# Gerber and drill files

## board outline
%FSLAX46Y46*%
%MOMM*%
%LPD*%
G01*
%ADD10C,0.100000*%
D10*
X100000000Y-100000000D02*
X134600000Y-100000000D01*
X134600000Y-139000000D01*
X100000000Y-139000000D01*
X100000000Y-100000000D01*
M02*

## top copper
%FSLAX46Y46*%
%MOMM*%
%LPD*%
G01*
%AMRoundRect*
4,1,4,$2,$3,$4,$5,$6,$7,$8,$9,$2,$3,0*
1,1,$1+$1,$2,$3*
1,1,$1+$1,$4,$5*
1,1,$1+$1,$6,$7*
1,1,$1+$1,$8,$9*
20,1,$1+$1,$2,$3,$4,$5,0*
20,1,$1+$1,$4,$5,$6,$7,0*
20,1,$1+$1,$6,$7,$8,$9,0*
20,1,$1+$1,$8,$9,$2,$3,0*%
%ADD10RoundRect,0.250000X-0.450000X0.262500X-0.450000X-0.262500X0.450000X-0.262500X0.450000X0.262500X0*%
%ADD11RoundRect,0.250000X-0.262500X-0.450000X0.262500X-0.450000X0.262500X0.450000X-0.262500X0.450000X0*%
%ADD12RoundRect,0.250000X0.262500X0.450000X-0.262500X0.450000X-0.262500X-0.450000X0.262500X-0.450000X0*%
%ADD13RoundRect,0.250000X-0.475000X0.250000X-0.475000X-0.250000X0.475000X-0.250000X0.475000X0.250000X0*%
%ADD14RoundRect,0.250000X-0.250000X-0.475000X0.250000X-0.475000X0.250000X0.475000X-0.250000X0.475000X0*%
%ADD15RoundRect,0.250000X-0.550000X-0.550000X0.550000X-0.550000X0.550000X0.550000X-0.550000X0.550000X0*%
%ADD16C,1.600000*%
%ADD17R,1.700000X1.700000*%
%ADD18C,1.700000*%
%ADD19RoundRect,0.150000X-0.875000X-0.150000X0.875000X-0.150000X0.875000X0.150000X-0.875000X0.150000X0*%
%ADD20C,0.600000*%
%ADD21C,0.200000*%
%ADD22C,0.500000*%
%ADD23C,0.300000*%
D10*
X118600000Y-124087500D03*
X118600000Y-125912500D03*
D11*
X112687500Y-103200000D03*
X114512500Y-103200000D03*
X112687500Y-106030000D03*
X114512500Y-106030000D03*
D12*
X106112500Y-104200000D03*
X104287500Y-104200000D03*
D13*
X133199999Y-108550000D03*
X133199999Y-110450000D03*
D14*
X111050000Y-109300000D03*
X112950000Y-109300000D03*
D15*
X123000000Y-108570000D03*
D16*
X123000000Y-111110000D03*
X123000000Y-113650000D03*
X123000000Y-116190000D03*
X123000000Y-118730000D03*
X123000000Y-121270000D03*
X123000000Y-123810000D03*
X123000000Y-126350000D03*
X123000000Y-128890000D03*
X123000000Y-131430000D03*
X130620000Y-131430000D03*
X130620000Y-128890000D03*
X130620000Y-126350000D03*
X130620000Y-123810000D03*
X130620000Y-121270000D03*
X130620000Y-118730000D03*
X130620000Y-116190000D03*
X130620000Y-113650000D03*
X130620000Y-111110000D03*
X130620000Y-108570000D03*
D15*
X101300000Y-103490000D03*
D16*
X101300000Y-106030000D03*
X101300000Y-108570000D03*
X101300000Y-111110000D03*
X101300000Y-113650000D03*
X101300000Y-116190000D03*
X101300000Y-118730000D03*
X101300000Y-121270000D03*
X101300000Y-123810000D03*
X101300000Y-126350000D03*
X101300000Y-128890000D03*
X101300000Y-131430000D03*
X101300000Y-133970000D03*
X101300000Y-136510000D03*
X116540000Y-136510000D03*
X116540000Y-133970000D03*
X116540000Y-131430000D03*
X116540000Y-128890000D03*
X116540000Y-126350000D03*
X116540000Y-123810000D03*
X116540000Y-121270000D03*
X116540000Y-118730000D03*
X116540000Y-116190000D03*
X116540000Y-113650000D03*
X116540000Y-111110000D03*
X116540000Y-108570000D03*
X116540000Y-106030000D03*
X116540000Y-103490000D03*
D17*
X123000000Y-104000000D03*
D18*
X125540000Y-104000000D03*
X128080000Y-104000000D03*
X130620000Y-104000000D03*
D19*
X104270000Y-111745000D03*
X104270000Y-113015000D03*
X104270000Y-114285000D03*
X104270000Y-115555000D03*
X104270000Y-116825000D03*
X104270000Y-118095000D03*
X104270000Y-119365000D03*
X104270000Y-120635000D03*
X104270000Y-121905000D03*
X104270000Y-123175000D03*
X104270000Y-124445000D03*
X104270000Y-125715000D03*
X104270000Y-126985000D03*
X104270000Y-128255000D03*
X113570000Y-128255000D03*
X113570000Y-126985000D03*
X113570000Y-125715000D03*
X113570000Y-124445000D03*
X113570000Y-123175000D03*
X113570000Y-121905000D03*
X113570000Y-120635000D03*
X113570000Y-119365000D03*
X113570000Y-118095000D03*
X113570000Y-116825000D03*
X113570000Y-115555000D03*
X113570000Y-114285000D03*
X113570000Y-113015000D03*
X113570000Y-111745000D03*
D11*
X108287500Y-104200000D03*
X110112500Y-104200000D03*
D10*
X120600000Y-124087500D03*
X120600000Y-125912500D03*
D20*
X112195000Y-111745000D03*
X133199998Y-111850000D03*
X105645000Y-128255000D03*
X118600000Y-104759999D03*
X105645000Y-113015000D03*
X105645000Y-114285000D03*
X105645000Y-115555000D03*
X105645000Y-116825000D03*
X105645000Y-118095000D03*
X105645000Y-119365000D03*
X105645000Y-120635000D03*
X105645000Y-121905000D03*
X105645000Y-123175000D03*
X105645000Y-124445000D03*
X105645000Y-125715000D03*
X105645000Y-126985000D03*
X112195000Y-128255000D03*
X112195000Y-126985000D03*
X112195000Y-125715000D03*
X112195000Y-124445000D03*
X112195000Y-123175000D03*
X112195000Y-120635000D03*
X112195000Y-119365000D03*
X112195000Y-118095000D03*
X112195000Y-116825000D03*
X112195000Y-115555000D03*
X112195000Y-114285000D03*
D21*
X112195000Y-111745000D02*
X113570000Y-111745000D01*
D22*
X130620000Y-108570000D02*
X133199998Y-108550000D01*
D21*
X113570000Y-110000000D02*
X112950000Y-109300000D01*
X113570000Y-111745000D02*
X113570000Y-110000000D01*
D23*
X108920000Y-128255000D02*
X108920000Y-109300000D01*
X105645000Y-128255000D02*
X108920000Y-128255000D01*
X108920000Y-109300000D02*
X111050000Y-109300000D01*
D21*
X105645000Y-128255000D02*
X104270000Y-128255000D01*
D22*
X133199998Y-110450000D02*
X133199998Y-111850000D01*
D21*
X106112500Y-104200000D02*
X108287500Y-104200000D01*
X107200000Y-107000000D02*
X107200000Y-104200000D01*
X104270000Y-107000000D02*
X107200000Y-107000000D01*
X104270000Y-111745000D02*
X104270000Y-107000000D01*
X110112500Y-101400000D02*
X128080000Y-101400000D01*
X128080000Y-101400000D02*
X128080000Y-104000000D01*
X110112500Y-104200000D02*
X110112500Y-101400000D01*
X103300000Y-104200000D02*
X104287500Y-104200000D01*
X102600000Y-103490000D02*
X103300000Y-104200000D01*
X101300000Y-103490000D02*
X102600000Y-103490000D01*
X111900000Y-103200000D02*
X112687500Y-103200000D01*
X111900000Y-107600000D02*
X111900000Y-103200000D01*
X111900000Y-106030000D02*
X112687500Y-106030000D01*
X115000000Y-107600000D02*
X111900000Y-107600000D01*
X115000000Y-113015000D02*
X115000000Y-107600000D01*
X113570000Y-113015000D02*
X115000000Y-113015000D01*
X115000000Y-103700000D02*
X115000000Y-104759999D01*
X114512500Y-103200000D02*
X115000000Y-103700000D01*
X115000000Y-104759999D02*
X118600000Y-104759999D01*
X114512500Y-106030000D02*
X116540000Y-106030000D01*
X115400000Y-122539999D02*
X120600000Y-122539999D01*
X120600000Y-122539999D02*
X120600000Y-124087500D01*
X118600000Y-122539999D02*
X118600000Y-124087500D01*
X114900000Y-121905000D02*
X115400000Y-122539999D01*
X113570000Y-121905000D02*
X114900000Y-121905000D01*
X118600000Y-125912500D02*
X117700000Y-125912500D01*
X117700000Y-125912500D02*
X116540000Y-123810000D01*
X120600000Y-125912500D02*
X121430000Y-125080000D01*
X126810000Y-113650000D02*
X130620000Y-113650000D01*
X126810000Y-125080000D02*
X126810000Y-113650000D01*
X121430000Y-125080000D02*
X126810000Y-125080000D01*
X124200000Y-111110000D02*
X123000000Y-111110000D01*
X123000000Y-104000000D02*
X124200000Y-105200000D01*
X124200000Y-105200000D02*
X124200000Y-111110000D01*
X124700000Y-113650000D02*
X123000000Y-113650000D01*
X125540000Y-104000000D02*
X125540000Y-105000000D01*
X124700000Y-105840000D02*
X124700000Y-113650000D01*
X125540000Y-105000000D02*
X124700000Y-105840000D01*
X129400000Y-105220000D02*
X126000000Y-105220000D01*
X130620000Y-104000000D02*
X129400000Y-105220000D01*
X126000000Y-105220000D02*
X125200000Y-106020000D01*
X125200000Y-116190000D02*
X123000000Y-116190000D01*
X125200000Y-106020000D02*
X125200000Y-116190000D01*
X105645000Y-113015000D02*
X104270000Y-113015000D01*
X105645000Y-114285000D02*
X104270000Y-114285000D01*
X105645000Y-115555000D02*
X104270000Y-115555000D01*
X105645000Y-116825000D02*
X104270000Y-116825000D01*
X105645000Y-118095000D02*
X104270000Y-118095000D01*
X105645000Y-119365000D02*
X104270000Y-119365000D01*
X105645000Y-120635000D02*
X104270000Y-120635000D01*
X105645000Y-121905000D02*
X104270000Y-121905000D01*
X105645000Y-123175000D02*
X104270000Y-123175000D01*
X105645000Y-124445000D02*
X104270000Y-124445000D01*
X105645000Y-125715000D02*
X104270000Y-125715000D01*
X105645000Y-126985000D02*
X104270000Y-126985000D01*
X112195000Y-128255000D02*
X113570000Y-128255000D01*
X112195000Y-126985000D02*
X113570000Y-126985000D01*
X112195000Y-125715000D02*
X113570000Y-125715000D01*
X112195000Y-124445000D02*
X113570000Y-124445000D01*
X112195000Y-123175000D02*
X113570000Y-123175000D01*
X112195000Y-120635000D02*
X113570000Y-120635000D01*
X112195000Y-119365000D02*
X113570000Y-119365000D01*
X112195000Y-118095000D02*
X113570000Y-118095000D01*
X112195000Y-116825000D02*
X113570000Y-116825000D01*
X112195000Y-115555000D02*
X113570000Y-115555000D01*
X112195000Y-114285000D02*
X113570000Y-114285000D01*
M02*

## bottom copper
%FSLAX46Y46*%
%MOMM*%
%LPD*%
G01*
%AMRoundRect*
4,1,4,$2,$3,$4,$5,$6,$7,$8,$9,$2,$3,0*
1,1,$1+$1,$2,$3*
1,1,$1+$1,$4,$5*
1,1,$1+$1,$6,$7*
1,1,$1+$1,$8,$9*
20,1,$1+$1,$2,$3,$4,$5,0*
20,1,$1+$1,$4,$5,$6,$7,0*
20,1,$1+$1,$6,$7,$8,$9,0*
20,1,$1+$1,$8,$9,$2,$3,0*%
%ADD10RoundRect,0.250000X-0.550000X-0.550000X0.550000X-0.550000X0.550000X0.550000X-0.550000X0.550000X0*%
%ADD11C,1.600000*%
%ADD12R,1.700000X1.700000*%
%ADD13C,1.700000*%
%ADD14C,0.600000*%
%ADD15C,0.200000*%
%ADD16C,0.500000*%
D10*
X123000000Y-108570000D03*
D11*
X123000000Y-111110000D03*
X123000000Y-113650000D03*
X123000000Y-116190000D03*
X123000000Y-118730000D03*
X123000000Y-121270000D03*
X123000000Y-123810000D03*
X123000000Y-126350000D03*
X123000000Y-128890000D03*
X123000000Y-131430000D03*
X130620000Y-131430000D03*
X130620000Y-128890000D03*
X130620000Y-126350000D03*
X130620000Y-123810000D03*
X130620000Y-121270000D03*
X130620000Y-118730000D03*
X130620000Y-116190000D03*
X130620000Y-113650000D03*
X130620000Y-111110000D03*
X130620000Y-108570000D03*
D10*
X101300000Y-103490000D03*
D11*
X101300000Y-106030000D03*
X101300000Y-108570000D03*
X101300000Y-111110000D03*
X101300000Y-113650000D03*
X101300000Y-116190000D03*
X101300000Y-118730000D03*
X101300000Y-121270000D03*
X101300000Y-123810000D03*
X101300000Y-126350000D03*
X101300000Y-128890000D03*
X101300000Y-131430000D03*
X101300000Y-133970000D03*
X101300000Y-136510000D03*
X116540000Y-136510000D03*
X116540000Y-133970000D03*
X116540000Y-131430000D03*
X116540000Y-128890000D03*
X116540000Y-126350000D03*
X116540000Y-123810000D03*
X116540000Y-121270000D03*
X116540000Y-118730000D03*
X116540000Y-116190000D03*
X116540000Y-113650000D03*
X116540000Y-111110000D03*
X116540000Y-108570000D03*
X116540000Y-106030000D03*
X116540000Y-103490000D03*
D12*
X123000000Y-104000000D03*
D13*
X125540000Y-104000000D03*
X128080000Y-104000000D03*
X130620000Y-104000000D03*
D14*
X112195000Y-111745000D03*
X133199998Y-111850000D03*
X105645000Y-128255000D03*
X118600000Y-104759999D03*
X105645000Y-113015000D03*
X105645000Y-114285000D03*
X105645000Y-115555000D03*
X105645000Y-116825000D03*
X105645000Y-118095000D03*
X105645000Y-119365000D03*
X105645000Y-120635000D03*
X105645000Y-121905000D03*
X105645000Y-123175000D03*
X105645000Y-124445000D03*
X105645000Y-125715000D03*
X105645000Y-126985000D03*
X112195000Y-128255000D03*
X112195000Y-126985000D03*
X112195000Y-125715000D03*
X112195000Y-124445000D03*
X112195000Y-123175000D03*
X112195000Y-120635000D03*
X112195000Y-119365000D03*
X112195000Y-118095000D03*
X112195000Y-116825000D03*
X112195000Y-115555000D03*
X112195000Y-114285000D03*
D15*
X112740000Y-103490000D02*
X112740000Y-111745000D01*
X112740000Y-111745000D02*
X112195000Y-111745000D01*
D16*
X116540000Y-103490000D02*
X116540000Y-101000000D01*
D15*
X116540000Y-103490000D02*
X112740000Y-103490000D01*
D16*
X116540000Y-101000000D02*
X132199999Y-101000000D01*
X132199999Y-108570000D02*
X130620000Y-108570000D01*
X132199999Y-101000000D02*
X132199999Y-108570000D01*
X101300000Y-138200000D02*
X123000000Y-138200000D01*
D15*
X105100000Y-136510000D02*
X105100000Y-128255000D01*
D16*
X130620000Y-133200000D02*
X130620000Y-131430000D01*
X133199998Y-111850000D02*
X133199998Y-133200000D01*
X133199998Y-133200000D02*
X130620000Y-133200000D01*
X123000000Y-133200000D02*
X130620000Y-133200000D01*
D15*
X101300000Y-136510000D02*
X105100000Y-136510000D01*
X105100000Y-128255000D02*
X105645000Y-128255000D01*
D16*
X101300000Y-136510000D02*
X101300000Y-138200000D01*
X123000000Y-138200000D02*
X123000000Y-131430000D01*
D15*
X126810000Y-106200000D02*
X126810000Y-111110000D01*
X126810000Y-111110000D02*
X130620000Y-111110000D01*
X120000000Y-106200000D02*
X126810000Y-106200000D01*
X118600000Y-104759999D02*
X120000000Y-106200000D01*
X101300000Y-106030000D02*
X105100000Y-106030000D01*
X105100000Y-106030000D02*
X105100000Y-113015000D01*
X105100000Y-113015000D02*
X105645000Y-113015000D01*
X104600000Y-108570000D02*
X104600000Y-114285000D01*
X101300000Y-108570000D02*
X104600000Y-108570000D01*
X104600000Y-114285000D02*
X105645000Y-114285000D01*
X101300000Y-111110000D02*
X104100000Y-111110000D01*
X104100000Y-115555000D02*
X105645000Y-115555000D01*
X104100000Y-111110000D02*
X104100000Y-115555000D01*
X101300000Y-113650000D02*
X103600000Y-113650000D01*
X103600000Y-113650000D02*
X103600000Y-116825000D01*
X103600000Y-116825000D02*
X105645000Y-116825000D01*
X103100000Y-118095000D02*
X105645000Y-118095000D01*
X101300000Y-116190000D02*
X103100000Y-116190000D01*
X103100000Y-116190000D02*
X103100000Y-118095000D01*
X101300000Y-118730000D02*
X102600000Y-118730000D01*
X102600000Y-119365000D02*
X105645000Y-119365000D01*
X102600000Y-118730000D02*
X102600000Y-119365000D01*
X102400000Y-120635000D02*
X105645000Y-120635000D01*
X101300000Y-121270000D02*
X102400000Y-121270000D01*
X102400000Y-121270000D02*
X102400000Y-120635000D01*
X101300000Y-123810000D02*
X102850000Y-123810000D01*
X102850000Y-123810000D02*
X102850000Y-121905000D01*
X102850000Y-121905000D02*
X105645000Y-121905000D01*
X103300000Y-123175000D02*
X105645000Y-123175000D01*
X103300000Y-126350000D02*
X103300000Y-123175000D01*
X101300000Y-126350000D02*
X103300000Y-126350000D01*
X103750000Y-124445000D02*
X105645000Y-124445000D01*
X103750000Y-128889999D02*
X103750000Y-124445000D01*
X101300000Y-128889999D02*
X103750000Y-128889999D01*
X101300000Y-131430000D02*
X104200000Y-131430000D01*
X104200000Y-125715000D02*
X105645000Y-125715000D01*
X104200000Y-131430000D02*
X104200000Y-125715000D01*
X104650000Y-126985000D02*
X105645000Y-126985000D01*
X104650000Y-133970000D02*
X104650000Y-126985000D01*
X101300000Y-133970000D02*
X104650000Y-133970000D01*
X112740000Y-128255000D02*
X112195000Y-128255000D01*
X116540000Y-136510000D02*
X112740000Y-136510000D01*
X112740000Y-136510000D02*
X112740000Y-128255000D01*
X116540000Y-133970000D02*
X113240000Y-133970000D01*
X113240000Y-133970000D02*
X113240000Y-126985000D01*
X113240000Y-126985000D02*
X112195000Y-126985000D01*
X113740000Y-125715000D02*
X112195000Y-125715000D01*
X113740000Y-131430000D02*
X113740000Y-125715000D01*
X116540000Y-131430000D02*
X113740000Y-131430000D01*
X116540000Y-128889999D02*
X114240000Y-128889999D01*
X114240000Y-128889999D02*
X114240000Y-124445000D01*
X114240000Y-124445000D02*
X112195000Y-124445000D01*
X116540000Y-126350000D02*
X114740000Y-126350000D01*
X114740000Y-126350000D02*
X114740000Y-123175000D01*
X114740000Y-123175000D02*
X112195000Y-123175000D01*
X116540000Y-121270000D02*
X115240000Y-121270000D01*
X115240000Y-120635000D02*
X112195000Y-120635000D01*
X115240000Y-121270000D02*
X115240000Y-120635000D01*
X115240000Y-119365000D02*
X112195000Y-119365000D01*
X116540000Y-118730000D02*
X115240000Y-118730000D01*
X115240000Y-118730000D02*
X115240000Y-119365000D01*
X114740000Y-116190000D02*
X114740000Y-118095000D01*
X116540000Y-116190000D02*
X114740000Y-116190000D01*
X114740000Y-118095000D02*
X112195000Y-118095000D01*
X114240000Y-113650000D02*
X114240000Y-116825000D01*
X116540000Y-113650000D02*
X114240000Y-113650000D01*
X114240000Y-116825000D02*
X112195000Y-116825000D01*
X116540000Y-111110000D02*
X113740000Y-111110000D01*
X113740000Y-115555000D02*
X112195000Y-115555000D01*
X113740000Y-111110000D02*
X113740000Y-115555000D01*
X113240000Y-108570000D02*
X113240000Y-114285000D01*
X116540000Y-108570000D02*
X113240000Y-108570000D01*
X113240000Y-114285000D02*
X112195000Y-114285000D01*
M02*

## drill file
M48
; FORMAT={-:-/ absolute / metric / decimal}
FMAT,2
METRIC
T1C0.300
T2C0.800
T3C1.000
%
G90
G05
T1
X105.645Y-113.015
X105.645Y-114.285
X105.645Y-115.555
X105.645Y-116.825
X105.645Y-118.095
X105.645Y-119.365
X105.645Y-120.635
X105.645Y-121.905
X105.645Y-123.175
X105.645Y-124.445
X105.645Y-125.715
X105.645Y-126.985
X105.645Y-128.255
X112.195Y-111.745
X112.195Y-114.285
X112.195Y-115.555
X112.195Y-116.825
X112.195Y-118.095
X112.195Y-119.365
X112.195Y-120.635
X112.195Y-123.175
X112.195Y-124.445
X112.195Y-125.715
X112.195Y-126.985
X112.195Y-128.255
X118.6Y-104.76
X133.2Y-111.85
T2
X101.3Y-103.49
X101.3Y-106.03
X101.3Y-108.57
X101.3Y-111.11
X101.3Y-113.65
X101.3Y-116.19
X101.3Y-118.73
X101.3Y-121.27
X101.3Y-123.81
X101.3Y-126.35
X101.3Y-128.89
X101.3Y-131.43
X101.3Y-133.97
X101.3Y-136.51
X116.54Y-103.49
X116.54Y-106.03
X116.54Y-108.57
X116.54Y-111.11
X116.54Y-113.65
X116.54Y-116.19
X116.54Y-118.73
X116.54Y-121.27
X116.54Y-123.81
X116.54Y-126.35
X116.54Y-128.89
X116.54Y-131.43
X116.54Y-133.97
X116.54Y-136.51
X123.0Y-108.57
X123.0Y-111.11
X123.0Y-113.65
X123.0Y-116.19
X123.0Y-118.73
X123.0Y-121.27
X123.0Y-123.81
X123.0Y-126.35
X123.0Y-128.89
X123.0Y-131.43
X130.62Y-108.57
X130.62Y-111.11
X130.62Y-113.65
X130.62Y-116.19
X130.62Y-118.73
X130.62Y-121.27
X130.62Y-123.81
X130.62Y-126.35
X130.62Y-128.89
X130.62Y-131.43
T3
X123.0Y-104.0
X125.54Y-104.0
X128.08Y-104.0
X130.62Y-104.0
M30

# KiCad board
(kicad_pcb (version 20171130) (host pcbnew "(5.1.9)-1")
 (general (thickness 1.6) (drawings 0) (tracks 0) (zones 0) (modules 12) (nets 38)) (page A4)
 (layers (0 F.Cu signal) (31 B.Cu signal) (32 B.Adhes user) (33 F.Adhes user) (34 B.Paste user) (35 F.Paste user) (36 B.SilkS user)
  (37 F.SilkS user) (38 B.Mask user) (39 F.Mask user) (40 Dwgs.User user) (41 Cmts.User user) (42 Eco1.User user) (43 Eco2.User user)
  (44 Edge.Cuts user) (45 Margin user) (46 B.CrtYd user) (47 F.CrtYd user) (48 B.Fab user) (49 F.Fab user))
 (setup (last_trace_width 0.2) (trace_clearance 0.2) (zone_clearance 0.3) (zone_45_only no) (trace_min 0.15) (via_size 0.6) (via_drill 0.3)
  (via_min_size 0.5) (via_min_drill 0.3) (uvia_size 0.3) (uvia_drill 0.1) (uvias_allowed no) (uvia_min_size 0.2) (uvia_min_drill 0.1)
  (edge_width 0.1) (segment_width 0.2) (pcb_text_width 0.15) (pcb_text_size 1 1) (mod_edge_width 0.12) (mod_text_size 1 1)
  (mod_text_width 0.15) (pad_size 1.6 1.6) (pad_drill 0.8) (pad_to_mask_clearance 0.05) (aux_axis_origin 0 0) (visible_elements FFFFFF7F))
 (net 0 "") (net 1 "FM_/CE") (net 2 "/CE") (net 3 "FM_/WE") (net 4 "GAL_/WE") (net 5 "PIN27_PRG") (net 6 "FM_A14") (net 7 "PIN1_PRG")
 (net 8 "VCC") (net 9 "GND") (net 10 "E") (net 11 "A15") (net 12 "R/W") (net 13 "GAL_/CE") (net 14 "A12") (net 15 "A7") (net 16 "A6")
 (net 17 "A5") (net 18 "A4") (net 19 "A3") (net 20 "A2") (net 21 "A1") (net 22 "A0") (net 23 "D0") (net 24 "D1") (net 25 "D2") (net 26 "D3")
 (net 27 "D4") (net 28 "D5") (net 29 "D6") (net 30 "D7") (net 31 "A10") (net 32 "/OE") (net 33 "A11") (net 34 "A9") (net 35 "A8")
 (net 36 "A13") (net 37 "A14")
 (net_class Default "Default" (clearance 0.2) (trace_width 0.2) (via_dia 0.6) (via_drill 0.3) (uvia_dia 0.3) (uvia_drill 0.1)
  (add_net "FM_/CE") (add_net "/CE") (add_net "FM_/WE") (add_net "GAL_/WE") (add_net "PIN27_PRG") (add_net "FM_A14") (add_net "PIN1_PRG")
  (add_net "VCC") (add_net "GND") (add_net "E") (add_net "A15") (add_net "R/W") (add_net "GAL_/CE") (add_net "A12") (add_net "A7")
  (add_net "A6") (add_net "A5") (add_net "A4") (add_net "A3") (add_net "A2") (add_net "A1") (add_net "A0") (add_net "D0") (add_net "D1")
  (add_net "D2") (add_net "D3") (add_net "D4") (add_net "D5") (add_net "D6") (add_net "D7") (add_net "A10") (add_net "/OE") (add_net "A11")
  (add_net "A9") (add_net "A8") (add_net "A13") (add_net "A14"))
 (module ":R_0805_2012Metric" (layer F.Cu) (at 118.6 125 -90)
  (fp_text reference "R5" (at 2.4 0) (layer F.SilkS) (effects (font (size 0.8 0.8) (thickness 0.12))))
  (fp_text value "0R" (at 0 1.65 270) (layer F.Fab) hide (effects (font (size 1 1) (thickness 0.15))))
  (pad "1" smd roundrect (at -0.9125 0 270) (size 1.025 1.4) (layers F.Cu F.Paste F.Mask) (roundrect_rratio 0.2439) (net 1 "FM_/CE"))
  (pad "2" smd roundrect (at 0.9125 0 270) (size 1.025 1.4) (layers F.Cu F.Paste F.Mask) (roundrect_rratio 0.2439) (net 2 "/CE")))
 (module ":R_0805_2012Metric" (layer F.Cu) (at 113.6 103.2)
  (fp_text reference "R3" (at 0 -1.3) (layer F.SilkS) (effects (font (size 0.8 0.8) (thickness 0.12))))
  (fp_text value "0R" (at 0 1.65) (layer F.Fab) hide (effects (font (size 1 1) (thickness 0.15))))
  (pad "1" smd roundrect (at -0.9125 0) (size 1.025 1.4) (layers F.Cu F.Paste F.Mask) (roundrect_rratio 0.2439) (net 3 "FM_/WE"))
  (pad "2" smd roundrect (at 0.9125 0) (size 1.025 1.4) (layers F.Cu F.Paste F.Mask) (roundrect_rratio 0.2439) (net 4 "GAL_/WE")))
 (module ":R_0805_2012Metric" (layer F.Cu) (at 113.6 106.03)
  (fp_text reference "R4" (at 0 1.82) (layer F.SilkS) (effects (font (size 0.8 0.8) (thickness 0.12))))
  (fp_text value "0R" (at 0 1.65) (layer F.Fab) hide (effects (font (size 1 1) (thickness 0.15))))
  (pad "1" smd roundrect (at -0.9125 0) (size 1.025 1.4) (layers F.Cu F.Paste F.Mask) (roundrect_rratio 0.2439) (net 3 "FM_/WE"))
  (pad "2" smd roundrect (at 0.9125 0) (size 1.025 1.4) (layers F.Cu F.Paste F.Mask) (roundrect_rratio 0.2439) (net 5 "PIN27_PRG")))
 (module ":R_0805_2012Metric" (layer F.Cu) (at 105.2 104.2 180)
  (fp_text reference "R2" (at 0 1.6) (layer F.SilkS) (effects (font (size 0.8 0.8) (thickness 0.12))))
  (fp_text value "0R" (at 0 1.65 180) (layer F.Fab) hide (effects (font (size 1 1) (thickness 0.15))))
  (pad "1" smd roundrect (at -0.9125 0 180) (size 1.025 1.4) (layers F.Cu F.Paste F.Mask) (roundrect_rratio 0.2439) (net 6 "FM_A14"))
  (pad "2" smd roundrect (at 0.9125 0 180) (size 1.025 1.4) (layers F.Cu F.Paste F.Mask) (roundrect_rratio 0.2439) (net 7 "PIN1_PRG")))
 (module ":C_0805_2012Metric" (layer F.Cu) (at 133.2 109.5 -90)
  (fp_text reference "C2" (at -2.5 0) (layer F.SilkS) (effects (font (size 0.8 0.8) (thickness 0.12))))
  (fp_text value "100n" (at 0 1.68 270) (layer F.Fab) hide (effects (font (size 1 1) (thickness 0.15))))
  (pad "1" smd roundrect (at -0.95 0 270) (size 1 1.45) (layers F.Cu F.Paste F.Mask) (roundrect_rratio 0.25) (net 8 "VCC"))
  (pad "2" smd roundrect (at 0.95 0 270) (size 1 1.45) (layers F.Cu F.Paste F.Mask) (roundrect_rratio 0.25) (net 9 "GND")))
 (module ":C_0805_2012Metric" (layer F.Cu) (at 112 109.3)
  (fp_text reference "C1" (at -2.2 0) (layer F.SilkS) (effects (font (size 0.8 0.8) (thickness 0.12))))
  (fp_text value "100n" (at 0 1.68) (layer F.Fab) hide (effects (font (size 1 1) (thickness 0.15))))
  (pad "1" smd roundrect (at -0.95 0) (size 1 1.45) (layers F.Cu F.Paste F.Mask) (roundrect_rratio 0.25) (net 9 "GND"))
  (pad "2" smd roundrect (at 0.95 0) (size 1 1.45) (layers F.Cu F.Paste F.Mask) (roundrect_rratio 0.25) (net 8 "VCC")))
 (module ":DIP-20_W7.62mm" (layer F.Cu) (at 123 108.57)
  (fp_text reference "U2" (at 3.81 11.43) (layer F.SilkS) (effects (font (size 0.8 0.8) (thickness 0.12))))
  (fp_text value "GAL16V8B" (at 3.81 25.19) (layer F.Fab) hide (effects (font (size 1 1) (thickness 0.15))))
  (pad "1" thru_hole roundrect (at 0 0) (size 1.6 1.6) (drill 0.8) (layers *.Cu *.Mask) (roundrect_rratio 0.1562))
  (pad "2" thru_hole circle (at 0 2.54) (size 1.6 1.6) (drill 0.8) (layers *.Cu *.Mask) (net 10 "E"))
  (pad "3" thru_hole circle (at 0 5.08) (size 1.6 1.6) (drill 0.8) (layers *.Cu *.Mask) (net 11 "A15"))
  (pad "4" thru_hole circle (at 0 7.62) (size 1.6 1.6) (drill 0.8) (layers *.Cu *.Mask) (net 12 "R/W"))
  (pad "5" thru_hole circle (at 0 10.16) (size 1.6 1.6) (drill 0.8) (layers *.Cu *.Mask))
  (pad "6" thru_hole circle (at 0 12.7) (size 1.6 1.6) (drill 0.8) (layers *.Cu *.Mask))
  (pad "7" thru_hole circle (at 0 15.24) (size 1.6 1.6) (drill 0.8) (layers *.Cu *.Mask))
  (pad "8" thru_hole circle (at 0 17.78) (size 1.6 1.6) (drill 0.8) (layers *.Cu *.Mask))
  (pad "9" thru_hole circle (at 0 20.32) (size 1.6 1.6) (drill 0.8) (layers *.Cu *.Mask))
  (pad "10" thru_hole circle (at 0 22.86) (size 1.6 1.6) (drill 0.8) (layers *.Cu *.Mask) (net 9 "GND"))
  (pad "11" thru_hole circle (at 7.62 22.86) (size 1.6 1.6) (drill 0.8) (layers *.Cu *.Mask) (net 9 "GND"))
  (pad "12" thru_hole circle (at 7.62 20.32) (size 1.6 1.6) (drill 0.8) (layers *.Cu *.Mask))
  (pad "13" thru_hole circle (at 7.62 17.78) (size 1.6 1.6) (drill 0.8) (layers *.Cu *.Mask))
  (pad "14" thru_hole circle (at 7.62 15.24) (size 1.6 1.6) (drill 0.8) (layers *.Cu *.Mask))
  (pad "15" thru_hole circle (at 7.62 12.7) (size 1.6 1.6) (drill 0.8) (layers *.Cu *.Mask))
  (pad "16" thru_hole circle (at 7.62 10.16) (size 1.6 1.6) (drill 0.8) (layers *.Cu *.Mask))
  (pad "17" thru_hole circle (at 7.62 7.62) (size 1.6 1.6) (drill 0.8) (layers *.Cu *.Mask))
  (pad "18" thru_hole circle (at 7.62 5.08) (size 1.6 1.6) (drill 0.8) (layers *.Cu *.Mask) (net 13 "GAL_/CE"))
  (pad "19" thru_hole circle (at 7.62 2.54) (size 1.6 1.6) (drill 0.8) (layers *.Cu *.Mask) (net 4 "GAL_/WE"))
  (pad "20" thru_hole circle (at 7.62 0) (size 1.6 1.6) (drill 0.8) (layers *.Cu *.Mask) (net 8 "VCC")))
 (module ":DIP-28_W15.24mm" (layer F.Cu) (at 101.3 103.49)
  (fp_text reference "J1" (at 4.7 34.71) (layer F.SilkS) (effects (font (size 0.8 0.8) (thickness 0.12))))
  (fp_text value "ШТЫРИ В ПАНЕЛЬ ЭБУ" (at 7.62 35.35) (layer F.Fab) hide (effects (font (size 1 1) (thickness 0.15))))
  (pad "1" thru_hole roundrect (at 0 0) (size 1.6 1.6) (drill 0.8) (layers *.Cu *.Mask) (roundrect_rratio 0.1562) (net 7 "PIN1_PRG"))
  (pad "2" thru_hole circle (at 0 2.54) (size 1.6 1.6) (drill 0.8) (layers *.Cu *.Mask) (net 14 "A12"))
  (pad "3" thru_hole circle (at 0 5.08) (size 1.6 1.6) (drill 0.8) (layers *.Cu *.Mask) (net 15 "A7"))
  (pad "4" thru_hole circle (at 0 7.62) (size 1.6 1.6) (drill 0.8) (layers *.Cu *.Mask) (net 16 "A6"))
  (pad "5" thru_hole circle (at 0 10.16) (size 1.6 1.6) (drill 0.8) (layers *.Cu *.Mask) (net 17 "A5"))
  (pad "6" thru_hole circle (at 0 12.7) (size 1.6 1.6) (drill 0.8) (layers *.Cu *.Mask) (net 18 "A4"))
  (pad "7" thru_hole circle (at 0 15.24) (size 1.6 1.6) (drill 0.8) (layers *.Cu *.Mask) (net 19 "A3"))
  (pad "8" thru_hole circle (at 0 17.78) (size 1.6 1.6) (drill 0.8) (layers *.Cu *.Mask) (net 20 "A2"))
  (pad "9" thru_hole circle (at 0 20.32) (size 1.6 1.6) (drill 0.8) (layers *.Cu *.Mask) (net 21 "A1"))
  (pad "10" thru_hole circle (at 0 22.86) (size 1.6 1.6) (drill 0.8) (layers *.Cu *.Mask) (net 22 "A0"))
  (pad "11" thru_hole circle (at 0 25.4) (size 1.6 1.6) (drill 0.8) (layers *.Cu *.Mask) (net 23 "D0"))
  (pad "12" thru_hole circle (at 0 27.94) (size 1.6 1.6) (drill 0.8) (layers *.Cu *.Mask) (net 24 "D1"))
  (pad "13" thru_hole circle (at 0 30.48) (size 1.6 1.6) (drill 0.8) (layers *.Cu *.Mask) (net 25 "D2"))
  (pad "14" thru_hole circle (at 0 33.02) (size 1.6 1.6) (drill 0.8) (layers *.Cu *.Mask) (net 9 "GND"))
  (pad "15" thru_hole circle (at 15.24 33.02) (size 1.6 1.6) (drill 0.8) (layers *.Cu *.Mask) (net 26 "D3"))
  (pad "16" thru_hole circle (at 15.24 30.48) (size 1.6 1.6) (drill 0.8) (layers *.Cu *.Mask) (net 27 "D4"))
  (pad "17" thru_hole circle (at 15.24 27.94) (size 1.6 1.6) (drill 0.8) (layers *.Cu *.Mask) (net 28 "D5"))
  (pad "18" thru_hole circle (at 15.24 25.4) (size 1.6 1.6) (drill 0.8) (layers *.Cu *.Mask) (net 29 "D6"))
  (pad "19" thru_hole circle (at 15.24 22.86) (size 1.6 1.6) (drill 0.8) (layers *.Cu *.Mask) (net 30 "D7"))
  (pad "20" thru_hole circle (at 15.24 20.32) (size 1.6 1.6) (drill 0.8) (layers *.Cu *.Mask) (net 2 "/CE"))
  (pad "21" thru_hole circle (at 15.24 17.78) (size 1.6 1.6) (drill 0.8) (layers *.Cu *.Mask) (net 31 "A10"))
  (pad "22" thru_hole circle (at 15.24 15.24) (size 1.6 1.6) (drill 0.8) (layers *.Cu *.Mask) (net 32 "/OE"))
  (pad "23" thru_hole circle (at 15.24 12.7) (size 1.6 1.6) (drill 0.8) (layers *.Cu *.Mask) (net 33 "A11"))
  (pad "24" thru_hole circle (at 15.24 10.16) (size 1.6 1.6) (drill 0.8) (layers *.Cu *.Mask) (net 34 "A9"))
  (pad "25" thru_hole circle (at 15.24 7.62) (size 1.6 1.6) (drill 0.8) (layers *.Cu *.Mask) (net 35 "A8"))
  (pad "26" thru_hole circle (at 15.24 5.08) (size 1.6 1.6) (drill 0.8) (layers *.Cu *.Mask) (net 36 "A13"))
  (pad "27" thru_hole circle (at 15.24 2.54) (size 1.6 1.6) (drill 0.8) (layers *.Cu *.Mask) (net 5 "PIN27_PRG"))
  (pad "28" thru_hole circle (at 15.24 0) (size 1.6 1.6) (drill 0.8) (layers *.Cu *.Mask) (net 8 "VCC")))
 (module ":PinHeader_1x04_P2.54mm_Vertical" (layer F.Cu) (at 123 104 90)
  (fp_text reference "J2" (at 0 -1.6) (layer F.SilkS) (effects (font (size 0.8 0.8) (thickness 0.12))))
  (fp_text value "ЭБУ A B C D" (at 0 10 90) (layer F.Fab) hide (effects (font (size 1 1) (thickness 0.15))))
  (pad "1" thru_hole rect (at 0 0 90) (size 1.7 1.7) (drill 1) (layers *.Cu *.Mask) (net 10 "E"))
  (pad "2" thru_hole circle (at 0 2.54 90) (size 1.7 1.7) (drill 1) (layers *.Cu *.Mask) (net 11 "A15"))
  (pad "3" thru_hole circle (at 0 5.08 90) (size 1.7 1.7) (drill 1) (layers *.Cu *.Mask) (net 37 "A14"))
  (pad "4" thru_hole circle (at 0 7.62 90) (size 1.7 1.7) (drill 1) (layers *.Cu *.Mask) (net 12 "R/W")))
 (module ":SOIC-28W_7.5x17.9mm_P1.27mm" (layer F.Cu) (at 108.92 120)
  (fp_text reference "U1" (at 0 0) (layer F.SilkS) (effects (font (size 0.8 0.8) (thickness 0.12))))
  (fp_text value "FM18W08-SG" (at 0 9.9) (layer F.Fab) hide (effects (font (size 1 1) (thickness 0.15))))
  (pad "1" smd roundrect (at -4.65 -8.255) (size 2.05 0.6) (layers F.Cu F.Paste F.Mask) (roundrect_rratio 0.25) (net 6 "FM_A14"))
  (pad "2" smd roundrect (at -4.65 -6.985) (size 2.05 0.6) (layers F.Cu F.Paste F.Mask) (roundrect_rratio 0.25) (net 14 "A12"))
  (pad "3" smd roundrect (at -4.65 -5.715) (size 2.05 0.6) (layers F.Cu F.Paste F.Mask) (roundrect_rratio 0.25) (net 15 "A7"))
  (pad "4" smd roundrect (at -4.65 -4.445) (size 2.05 0.6) (layers F.Cu F.Paste F.Mask) (roundrect_rratio 0.25) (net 16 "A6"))
  (pad "5" smd roundrect (at -4.65 -3.175) (size 2.05 0.6) (layers F.Cu F.Paste F.Mask) (roundrect_rratio 0.25) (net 17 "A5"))
  (pad "6" smd roundrect (at -4.65 -1.905) (size 2.05 0.6) (layers F.Cu F.Paste F.Mask) (roundrect_rratio 0.25) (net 18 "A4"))
  (pad "7" smd roundrect (at -4.65 -0.635) (size 2.05 0.6) (layers F.Cu F.Paste F.Mask) (roundrect_rratio 0.25) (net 19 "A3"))
  (pad "8" smd roundrect (at -4.65 0.635) (size 2.05 0.6) (layers F.Cu F.Paste F.Mask) (roundrect_rratio 0.25) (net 20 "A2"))
  (pad "9" smd roundrect (at -4.65 1.905) (size 2.05 0.6) (layers F.Cu F.Paste F.Mask) (roundrect_rratio 0.25) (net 21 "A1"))
  (pad "10" smd roundrect (at -4.65 3.175) (size 2.05 0.6) (layers F.Cu F.Paste F.Mask) (roundrect_rratio 0.25) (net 22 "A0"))
  (pad "11" smd roundrect (at -4.65 4.445) (size 2.05 0.6) (layers F.Cu F.Paste F.Mask) (roundrect_rratio 0.25) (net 23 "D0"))
  (pad "12" smd roundrect (at -4.65 5.715) (size 2.05 0.6) (layers F.Cu F.Paste F.Mask) (roundrect_rratio 0.25) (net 24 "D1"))
  (pad "13" smd roundrect (at -4.65 6.985) (size 2.05 0.6) (layers F.Cu F.Paste F.Mask) (roundrect_rratio 0.25) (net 25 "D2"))
  (pad "14" smd roundrect (at -4.65 8.255) (size 2.05 0.6) (layers F.Cu F.Paste F.Mask) (roundrect_rratio 0.25) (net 9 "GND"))
  (pad "15" smd roundrect (at 4.65 8.255) (size 2.05 0.6) (layers F.Cu F.Paste F.Mask) (roundrect_rratio 0.25) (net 26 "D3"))
  (pad "16" smd roundrect (at 4.65 6.985) (size 2.05 0.6) (layers F.Cu F.Paste F.Mask) (roundrect_rratio 0.25) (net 27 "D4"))
  (pad "17" smd roundrect (at 4.65 5.715) (size 2.05 0.6) (layers F.Cu F.Paste F.Mask) (roundrect_rratio 0.25) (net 28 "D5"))
  (pad "18" smd roundrect (at 4.65 4.445) (size 2.05 0.6) (layers F.Cu F.Paste F.Mask) (roundrect_rratio 0.25) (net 29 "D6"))
  (pad "19" smd roundrect (at 4.65 3.175) (size 2.05 0.6) (layers F.Cu F.Paste F.Mask) (roundrect_rratio 0.25) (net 30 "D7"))
  (pad "20" smd roundrect (at 4.65 1.905) (size 2.05 0.6) (layers F.Cu F.Paste F.Mask) (roundrect_rratio 0.25) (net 1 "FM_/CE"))
  (pad "21" smd roundrect (at 4.65 0.635) (size 2.05 0.6) (layers F.Cu F.Paste F.Mask) (roundrect_rratio 0.25) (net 31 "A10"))
  (pad "22" smd roundrect (at 4.65 -0.635) (size 2.05 0.6) (layers F.Cu F.Paste F.Mask) (roundrect_rratio 0.25) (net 32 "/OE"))
  (pad "23" smd roundrect (at 4.65 -1.905) (size 2.05 0.6) (layers F.Cu F.Paste F.Mask) (roundrect_rratio 0.25) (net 33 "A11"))
  (pad "24" smd roundrect (at 4.65 -3.175) (size 2.05 0.6) (layers F.Cu F.Paste F.Mask) (roundrect_rratio 0.25) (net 34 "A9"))
  (pad "25" smd roundrect (at 4.65 -4.445) (size 2.05 0.6) (layers F.Cu F.Paste F.Mask) (roundrect_rratio 0.25) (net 35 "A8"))
  (pad "26" smd roundrect (at 4.65 -5.715) (size 2.05 0.6) (layers F.Cu F.Paste F.Mask) (roundrect_rratio 0.25) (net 36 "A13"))
  (pad "27" smd roundrect (at 4.65 -6.985) (size 2.05 0.6) (layers F.Cu F.Paste F.Mask) (roundrect_rratio 0.25) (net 3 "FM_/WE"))
  (pad "28" smd roundrect (at 4.65 -8.255) (size 2.05 0.6) (layers F.Cu F.Paste F.Mask) (roundrect_rratio 0.25) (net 8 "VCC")))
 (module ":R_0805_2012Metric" (layer F.Cu) (at 109.2 104.2)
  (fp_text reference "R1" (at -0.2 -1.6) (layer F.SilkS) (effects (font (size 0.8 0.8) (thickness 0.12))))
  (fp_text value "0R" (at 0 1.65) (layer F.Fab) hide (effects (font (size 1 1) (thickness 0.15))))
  (pad "1" smd roundrect (at -0.9125 0) (size 1.025 1.4) (layers F.Cu F.Paste F.Mask) (roundrect_rratio 0.2439) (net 6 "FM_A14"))
  (pad "2" smd roundrect (at 0.9125 0) (size 1.025 1.4) (layers F.Cu F.Paste F.Mask) (roundrect_rratio 0.2439) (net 37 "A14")))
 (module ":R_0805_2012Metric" (layer F.Cu) (at 120.6 125 -90)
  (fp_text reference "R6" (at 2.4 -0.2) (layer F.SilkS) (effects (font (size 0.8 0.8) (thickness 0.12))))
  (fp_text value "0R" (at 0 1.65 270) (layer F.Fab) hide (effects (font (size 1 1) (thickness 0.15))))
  (pad "1" smd roundrect (at -0.9125 0 270) (size 1.025 1.4) (layers F.Cu F.Paste F.Mask) (roundrect_rratio 0.2439) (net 1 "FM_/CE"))
  (pad "2" smd roundrect (at 0.9125 0 270) (size 1.025 1.4) (layers F.Cu F.Paste F.Mask) (roundrect_rratio 0.2439) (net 13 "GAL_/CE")))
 (gr_line (start 100 100) (end 134.6 100) (layer Edge.Cuts) (width 0.1))
 (gr_line (start 134.6 100) (end 134.6 139) (layer Edge.Cuts) (width 0.1))
 (gr_line (start 134.6 139) (end 100 139) (layer Edge.Cuts) (width 0.1))
 (gr_line (start 100 139) (end 100 100) (layer Edge.Cuts) (width 0.1))
 (segment (start 112.195 111.745) (end 113.57 111.745) (width 0.2) (layer F.Cu) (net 8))
 (segment (start 130.62 108.57) (end 133.2 108.55) (width 0.5) (layer F.Cu) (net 8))
 (segment (start 113.57 110) (end 112.95 109.3) (width 0.2) (layer F.Cu) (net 8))
 (segment (start 113.57 111.745) (end 113.57 110) (width 0.2) (layer F.Cu) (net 8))
 (via (at 112.195 111.745) (size 0.6) (drill 0.3) (layers F.Cu B.Cu) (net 8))
 (segment (start 112.74 103.49) (end 112.74 111.745) (width 0.2) (layer B.Cu) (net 8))
 (segment (start 112.74 111.745) (end 112.195 111.745) (width 0.2) (layer B.Cu) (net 8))
 (segment (start 116.54 103.49) (end 116.54 101) (width 0.5) (layer B.Cu) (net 8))
 (segment (start 116.54 103.49) (end 112.74 103.49) (width 0.2) (layer B.Cu) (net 8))
 (segment (start 116.54 101) (end 132.2 101) (width 0.5) (layer B.Cu) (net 8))
 (segment (start 132.2 108.57) (end 130.62 108.57) (width 0.5) (layer B.Cu) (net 8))
 (segment (start 132.2 101) (end 132.2 108.57) (width 0.5) (layer B.Cu) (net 8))
 (segment (start 108.92 128.255) (end 108.92 109.3) (width 0.3) (layer F.Cu) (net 9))
 (segment (start 105.645 128.255) (end 108.92 128.255) (width 0.3) (layer F.Cu) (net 9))
 (segment (start 108.92 109.3) (end 111.05 109.3) (width 0.3) (layer F.Cu) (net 9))
 (segment (start 105.645 128.255) (end 104.27 128.255) (width 0.2) (layer F.Cu) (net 9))
 (segment (start 133.2 110.45) (end 133.2 111.85) (width 0.5) (layer F.Cu) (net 9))
 (via (at 133.2 111.85) (size 0.6) (drill 0.3) (layers F.Cu B.Cu) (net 9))
 (via (at 105.645 128.255) (size 0.6) (drill 0.3) (layers F.Cu B.Cu) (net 9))
 (segment (start 101.3 138.2) (end 123 138.2) (width 0.5) (layer B.Cu) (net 9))
 (segment (start 105.1 136.51) (end 105.1 128.255) (width 0.2) (layer B.Cu) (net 9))
 (segment (start 130.62 133.2) (end 130.62 131.43) (width 0.5) (layer B.Cu) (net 9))
 (segment (start 133.2 111.85) (end 133.2 133.2) (width 0.5) (layer B.Cu) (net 9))
 (segment (start 133.2 133.2) (end 130.62 133.2) (width 0.5) (layer B.Cu) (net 9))
 (segment (start 123 133.2) (end 130.62 133.2) (width 0.5) (layer B.Cu) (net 9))
 (segment (start 101.3 136.51) (end 105.1 136.51) (width 0.2) (layer B.Cu) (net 9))
 (segment (start 105.1 128.255) (end 105.645 128.255) (width 0.2) (layer B.Cu) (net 9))
 (segment (start 101.3 136.51) (end 101.3 138.2) (width 0.5) (layer B.Cu) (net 9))
 (segment (start 123 138.2) (end 123 131.43) (width 0.5) (layer B.Cu) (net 9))
 (segment (start 106.1125 104.2) (end 108.2875 104.2) (width 0.2) (layer F.Cu) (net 6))
 (segment (start 107.2 107) (end 107.2 104.2) (width 0.2) (layer F.Cu) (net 6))
 (segment (start 104.27 107) (end 107.2 107) (width 0.2) (layer F.Cu) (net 6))
 (segment (start 104.27 111.745) (end 104.27 107) (width 0.2) (layer F.Cu) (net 6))
 (segment (start 110.1125 101.4) (end 128.08 101.4) (width 0.2) (layer F.Cu) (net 37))
 (segment (start 128.08 101.4) (end 128.08 104) (width 0.2) (layer F.Cu) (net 37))
 (segment (start 110.1125 104.2) (end 110.1125 101.4) (width 0.2) (layer F.Cu) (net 37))
 (segment (start 103.3 104.2) (end 104.2875 104.2) (width 0.2) (layer F.Cu) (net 7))
 (segment (start 102.6 103.49) (end 103.3 104.2) (width 0.2) (layer F.Cu) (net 7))
 (segment (start 101.3 103.49) (end 102.6 103.49) (width 0.2) (layer F.Cu) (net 7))
 (segment (start 111.9 103.2) (end 112.6875 103.2) (width 0.2) (layer F.Cu) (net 3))
 (segment (start 111.9 107.6) (end 111.9 103.2) (width 0.2) (layer F.Cu) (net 3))
 (segment (start 111.9 106.03) (end 112.6875 106.03) (width 0.2) (layer F.Cu) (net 3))
 (segment (start 115 107.6) (end 111.9 107.6) (width 0.2) (layer F.Cu) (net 3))
 (segment (start 115 113.015) (end 115 107.6) (width 0.2) (layer F.Cu) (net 3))
 (segment (start 113.57 113.015) (end 115 113.015) (width 0.2) (layer F.Cu) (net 3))
 (segment (start 115 103.7) (end 115 104.76) (width 0.2) (layer F.Cu) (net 4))
 (segment (start 114.5125 103.2) (end 115 103.7) (width 0.2) (layer F.Cu) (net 4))
 (segment (start 115 104.76) (end 118.6 104.76) (width 0.2) (layer F.Cu) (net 4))
 (via (at 118.6 104.76) (size 0.6) (drill 0.3) (layers F.Cu B.Cu) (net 4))
 (segment (start 126.81 106.2) (end 126.81 111.11) (width 0.2) (layer B.Cu) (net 4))
 (segment (start 126.81 111.11) (end 130.62 111.11) (width 0.2) (layer B.Cu) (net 4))
 (segment (start 120 106.2) (end 126.81 106.2) (width 0.2) (layer B.Cu) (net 4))
 (segment (start 118.6 104.76) (end 120 106.2) (width 0.2) (layer B.Cu) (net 4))
 (segment (start 114.5125 106.03) (end 116.54 106.03) (width 0.2) (layer F.Cu) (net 5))
 (segment (start 115.4 122.54) (end 120.6 122.54) (width 0.2) (layer F.Cu) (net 1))
 (segment (start 120.6 122.54) (end 120.6 124.0875) (width 0.2) (layer F.Cu) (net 1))
 (segment (start 118.6 122.54) (end 118.6 124.0875) (width 0.2) (layer F.Cu) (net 1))
 (segment (start 114.9 121.905) (end 115.4 122.54) (width 0.2) (layer F.Cu) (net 1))
 (segment (start 113.57 121.905) (end 114.9 121.905) (width 0.2) (layer F.Cu) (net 1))
 (segment (start 118.6 125.9125) (end 117.7 125.9125) (width 0.2) (layer F.Cu) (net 2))
 (segment (start 117.7 125.9125) (end 116.54 123.81) (width 0.2) (layer F.Cu) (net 2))
 (segment (start 120.6 125.9125) (end 121.43 125.08) (width 0.2) (layer F.Cu) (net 13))
 (segment (start 126.81 113.65) (end 130.62 113.65) (width 0.2) (layer F.Cu) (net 13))
 (segment (start 126.81 125.08) (end 126.81 113.65) (width 0.2) (layer F.Cu) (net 13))
 (segment (start 121.43 125.08) (end 126.81 125.08) (width 0.2) (layer F.Cu) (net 13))
 (segment (start 124.2 111.11) (end 123 111.11) (width 0.2) (layer F.Cu) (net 10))
 (segment (start 123 104) (end 124.2 105.2) (width 0.2) (layer F.Cu) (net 10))
 (segment (start 124.2 105.2) (end 124.2 111.11) (width 0.2) (layer F.Cu) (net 10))
 (segment (start 124.7 113.65) (end 123 113.65) (width 0.2) (layer F.Cu) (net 11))
 (segment (start 125.54 104) (end 125.54 105) (width 0.2) (layer F.Cu) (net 11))
 (segment (start 124.7 105.84) (end 124.7 113.65) (width 0.2) (layer F.Cu) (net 11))
 (segment (start 125.54 105) (end 124.7 105.84) (width 0.2) (layer F.Cu) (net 11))
 (segment (start 129.4 105.22) (end 126 105.22) (width 0.2) (layer F.Cu) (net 12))
 (segment (start 130.62 104) (end 129.4 105.22) (width 0.2) (layer F.Cu) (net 12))
 (segment (start 126 105.22) (end 125.2 106.02) (width 0.2) (layer F.Cu) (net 12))
 (segment (start 125.2 116.19) (end 123 116.19) (width 0.2) (layer F.Cu) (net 12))
 (segment (start 125.2 106.02) (end 125.2 116.19) (width 0.2) (layer F.Cu) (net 12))
 (segment (start 105.645 113.015) (end 104.27 113.015) (width 0.2) (layer F.Cu) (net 14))
 (via (at 105.645 113.015) (size 0.6) (drill 0.3) (layers F.Cu B.Cu) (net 14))
 (segment (start 101.3 106.03) (end 105.1 106.03) (width 0.2) (layer B.Cu) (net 14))
 (segment (start 105.1 106.03) (end 105.1 113.015) (width 0.2) (layer B.Cu) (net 14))
 (segment (start 105.1 113.015) (end 105.645 113.015) (width 0.2) (layer B.Cu) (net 14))
 (segment (start 105.645 114.285) (end 104.27 114.285) (width 0.2) (layer F.Cu) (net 15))
 (via (at 105.645 114.285) (size 0.6) (drill 0.3) (layers F.Cu B.Cu) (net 15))
 (segment (start 104.6 108.57) (end 104.6 114.285) (width 0.2) (layer B.Cu) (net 15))
 (segment (start 101.3 108.57) (end 104.6 108.57) (width 0.2) (layer B.Cu) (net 15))
 (segment (start 104.6 114.285) (end 105.645 114.285) (width 0.2) (layer B.Cu) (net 15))
 (segment (start 105.645 115.555) (end 104.27 115.555) (width 0.2) (layer F.Cu) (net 16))
 (via (at 105.645 115.555) (size 0.6) (drill 0.3) (layers F.Cu B.Cu) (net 16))
 (segment (start 101.3 111.11) (end 104.1 111.11) (width 0.2) (layer B.Cu) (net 16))
 (segment (start 104.1 115.555) (end 105.645 115.555) (width 0.2) (layer B.Cu) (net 16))
 (segment (start 104.1 111.11) (end 104.1 115.555) (width 0.2) (layer B.Cu) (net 16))
 (segment (start 105.645 116.825) (end 104.27 116.825) (width 0.2) (layer F.Cu) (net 17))
 (via (at 105.645 116.825) (size 0.6) (drill 0.3) (layers F.Cu B.Cu) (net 17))
 (segment (start 101.3 113.65) (end 103.6 113.65) (width 0.2) (layer B.Cu) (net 17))
 (segment (start 103.6 113.65) (end 103.6 116.825) (width 0.2) (layer B.Cu) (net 17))
 (segment (start 103.6 116.825) (end 105.645 116.825) (width 0.2) (layer B.Cu) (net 17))
 (segment (start 105.645 118.095) (end 104.27 118.095) (width 0.2) (layer F.Cu) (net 18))
 (via (at 105.645 118.095) (size 0.6) (drill 0.3) (layers F.Cu B.Cu) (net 18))
 (segment (start 103.1 118.095) (end 105.645 118.095) (width 0.2) (layer B.Cu) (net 18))
 (segment (start 101.3 116.19) (end 103.1 116.19) (width 0.2) (layer B.Cu) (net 18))
 (segment (start 103.1 116.19) (end 103.1 118.095) (width 0.2) (layer B.Cu) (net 18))
 (segment (start 105.645 119.365) (end 104.27 119.365) (width 0.2) (layer F.Cu) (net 19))
 (via (at 105.645 119.365) (size 0.6) (drill 0.3) (layers F.Cu B.Cu) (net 19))
 (segment (start 101.3 118.73) (end 102.6 118.73) (width 0.2) (layer B.Cu) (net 19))
 (segment (start 102.6 119.365) (end 105.645 119.365) (width 0.2) (layer B.Cu) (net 19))
 (segment (start 102.6 118.73) (end 102.6 119.365) (width 0.2) (layer B.Cu) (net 19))
 (segment (start 105.645 120.635) (end 104.27 120.635) (width 0.2) (layer F.Cu) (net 20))
 (via (at 105.645 120.635) (size 0.6) (drill 0.3) (layers F.Cu B.Cu) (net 20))
 (segment (start 102.4 120.635) (end 105.645 120.635) (width 0.2) (layer B.Cu) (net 20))
 (segment (start 101.3 121.27) (end 102.4 121.27) (width 0.2) (layer B.Cu) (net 20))
 (segment (start 102.4 121.27) (end 102.4 120.635) (width 0.2) (layer B.Cu) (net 20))
 (segment (start 105.645 121.905) (end 104.27 121.905) (width 0.2) (layer F.Cu) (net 21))
 (via (at 105.645 121.905) (size 0.6) (drill 0.3) (layers F.Cu B.Cu) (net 21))
 (segment (start 101.3 123.81) (end 102.85 123.81) (width 0.2) (layer B.Cu) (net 21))
 (segment (start 102.85 123.81) (end 102.85 121.905) (width 0.2) (layer B.Cu) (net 21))
 (segment (start 102.85 121.905) (end 105.645 121.905) (width 0.2) (layer B.Cu) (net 21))
 (segment (start 105.645 123.175) (end 104.27 123.175) (width 0.2) (layer F.Cu) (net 22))
 (via (at 105.645 123.175) (size 0.6) (drill 0.3) (layers F.Cu B.Cu) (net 22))
 (segment (start 103.3 123.175) (end 105.645 123.175) (width 0.2) (layer B.Cu) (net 22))
 (segment (start 103.3 126.35) (end 103.3 123.175) (width 0.2) (layer B.Cu) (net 22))
 (segment (start 101.3 126.35) (end 103.3 126.35) (width 0.2) (layer B.Cu) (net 22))
 (segment (start 105.645 124.445) (end 104.27 124.445) (width 0.2) (layer F.Cu) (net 23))
 (via (at 105.645 124.445) (size 0.6) (drill 0.3) (layers F.Cu B.Cu) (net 23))
 (segment (start 103.75 124.445) (end 105.645 124.445) (width 0.2) (layer B.Cu) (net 23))
 (segment (start 103.75 128.89) (end 103.75 124.445) (width 0.2) (layer B.Cu) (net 23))
 (segment (start 101.3 128.89) (end 103.75 128.89) (width 0.2) (layer B.Cu) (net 23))
 (segment (start 105.645 125.715) (end 104.27 125.715) (width 0.2) (layer F.Cu) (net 24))
 (via (at 105.645 125.715) (size 0.6) (drill 0.3) (layers F.Cu B.Cu) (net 24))
 (segment (start 101.3 131.43) (end 104.2 131.43) (width 0.2) (layer B.Cu) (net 24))
 (segment (start 104.2 125.715) (end 105.645 125.715) (width 0.2) (layer B.Cu) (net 24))
 (segment (start 104.2 131.43) (end 104.2 125.715) (width 0.2) (layer B.Cu) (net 24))
 (segment (start 105.645 126.985) (end 104.27 126.985) (width 0.2) (layer F.Cu) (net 25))
 (via (at 105.645 126.985) (size 0.6) (drill 0.3) (layers F.Cu B.Cu) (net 25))
 (segment (start 104.65 126.985) (end 105.645 126.985) (width 0.2) (layer B.Cu) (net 25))
 (segment (start 104.65 133.97) (end 104.65 126.985) (width 0.2) (layer B.Cu) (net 25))
 (segment (start 101.3 133.97) (end 104.65 133.97) (width 0.2) (layer B.Cu) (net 25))
 (segment (start 112.195 128.255) (end 113.57 128.255) (width 0.2) (layer F.Cu) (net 26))
 (via (at 112.195 128.255) (size 0.6) (drill 0.3) (layers F.Cu B.Cu) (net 26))
 (segment (start 112.74 128.255) (end 112.195 128.255) (width 0.2) (layer B.Cu) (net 26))
 (segment (start 116.54 136.51) (end 112.74 136.51) (width 0.2) (layer B.Cu) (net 26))
 (segment (start 112.74 136.51) (end 112.74 128.255) (width 0.2) (layer B.Cu) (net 26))
 (segment (start 112.195 126.985) (end 113.57 126.985) (width 0.2) (layer F.Cu) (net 27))
 (via (at 112.195 126.985) (size 0.6) (drill 0.3) (layers F.Cu B.Cu) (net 27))
 (segment (start 116.54 133.97) (end 113.24 133.97) (width 0.2) (layer B.Cu) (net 27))
 (segment (start 113.24 133.97) (end 113.24 126.985) (width 0.2) (layer B.Cu) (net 27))
 (segment (start 113.24 126.985) (end 112.195 126.985) (width 0.2) (layer B.Cu) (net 27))
 (segment (start 112.195 125.715) (end 113.57 125.715) (width 0.2) (layer F.Cu) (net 28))
 (via (at 112.195 125.715) (size 0.6) (drill 0.3) (layers F.Cu B.Cu) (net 28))
 (segment (start 113.74 125.715) (end 112.195 125.715) (width 0.2) (layer B.Cu) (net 28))
 (segment (start 113.74 131.43) (end 113.74 125.715) (width 0.2) (layer B.Cu) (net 28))
 (segment (start 116.54 131.43) (end 113.74 131.43) (width 0.2) (layer B.Cu) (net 28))
 (segment (start 112.195 124.445) (end 113.57 124.445) (width 0.2) (layer F.Cu) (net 29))
 (via (at 112.195 124.445) (size 0.6) (drill 0.3) (layers F.Cu B.Cu) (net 29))
 (segment (start 116.54 128.89) (end 114.24 128.89) (width 0.2) (layer B.Cu) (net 29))
 (segment (start 114.24 128.89) (end 114.24 124.445) (width 0.2) (layer B.Cu) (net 29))
 (segment (start 114.24 124.445) (end 112.195 124.445) (width 0.2) (layer B.Cu) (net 29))
 (segment (start 112.195 123.175) (end 113.57 123.175) (width 0.2) (layer F.Cu) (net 30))
 (via (at 112.195 123.175) (size 0.6) (drill 0.3) (layers F.Cu B.Cu) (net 30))
 (segment (start 116.54 126.35) (end 114.74 126.35) (width 0.2) (layer B.Cu) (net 30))
 (segment (start 114.74 126.35) (end 114.74 123.175) (width 0.2) (layer B.Cu) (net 30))
 (segment (start 114.74 123.175) (end 112.195 123.175) (width 0.2) (layer B.Cu) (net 30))
 (segment (start 112.195 120.635) (end 113.57 120.635) (width 0.2) (layer F.Cu) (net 31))
 (via (at 112.195 120.635) (size 0.6) (drill 0.3) (layers F.Cu B.Cu) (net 31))
 (segment (start 116.54 121.27) (end 115.24 121.27) (width 0.2) (layer B.Cu) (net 31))
 (segment (start 115.24 120.635) (end 112.195 120.635) (width 0.2) (layer B.Cu) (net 31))
 (segment (start 115.24 121.27) (end 115.24 120.635) (width 0.2) (layer B.Cu) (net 31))
 (segment (start 112.195 119.365) (end 113.57 119.365) (width 0.2) (layer F.Cu) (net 32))
 (via (at 112.195 119.365) (size 0.6) (drill 0.3) (layers F.Cu B.Cu) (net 32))
 (segment (start 115.24 119.365) (end 112.195 119.365) (width 0.2) (layer B.Cu) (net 32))
 (segment (start 116.54 118.73) (end 115.24 118.73) (width 0.2) (layer B.Cu) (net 32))
 (segment (start 115.24 118.73) (end 115.24 119.365) (width 0.2) (layer B.Cu) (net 32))
 (segment (start 112.195 118.095) (end 113.57 118.095) (width 0.2) (layer F.Cu) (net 33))
 (via (at 112.195 118.095) (size 0.6) (drill 0.3) (layers F.Cu B.Cu) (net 33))
 (segment (start 114.74 116.19) (end 114.74 118.095) (width 0.2) (layer B.Cu) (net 33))
 (segment (start 116.54 116.19) (end 114.74 116.19) (width 0.2) (layer B.Cu) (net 33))
 (segment (start 114.74 118.095) (end 112.195 118.095) (width 0.2) (layer B.Cu) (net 33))
 (segment (start 112.195 116.825) (end 113.57 116.825) (width 0.2) (layer F.Cu) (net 34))
 (via (at 112.195 116.825) (size 0.6) (drill 0.3) (layers F.Cu B.Cu) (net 34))
 (segment (start 114.24 113.65) (end 114.24 116.825) (width 0.2) (layer B.Cu) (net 34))
 (segment (start 116.54 113.65) (end 114.24 113.65) (width 0.2) (layer B.Cu) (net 34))
 (segment (start 114.24 116.825) (end 112.195 116.825) (width 0.2) (layer B.Cu) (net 34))
 (segment (start 112.195 115.555) (end 113.57 115.555) (width 0.2) (layer F.Cu) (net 35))
 (via (at 112.195 115.555) (size 0.6) (drill 0.3) (layers F.Cu B.Cu) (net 35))
 (segment (start 116.54 111.11) (end 113.74 111.11) (width 0.2) (layer B.Cu) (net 35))
 (segment (start 113.74 115.555) (end 112.195 115.555) (width 0.2) (layer B.Cu) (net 35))
 (segment (start 113.74 111.11) (end 113.74 115.555) (width 0.2) (layer B.Cu) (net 35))
 (segment (start 112.195 114.285) (end 113.57 114.285) (width 0.2) (layer F.Cu) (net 36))
 (via (at 112.195 114.285) (size 0.6) (drill 0.3) (layers F.Cu B.Cu) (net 36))
 (segment (start 113.24 108.57) (end 113.24 114.285) (width 0.2) (layer B.Cu) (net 36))
 (segment (start 116.54 108.57) (end 113.24 108.57) (width 0.2) (layer B.Cu) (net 36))
 (segment (start 113.24 114.285) (end 112.195 114.285) (width 0.2) (layer B.Cu) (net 36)))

